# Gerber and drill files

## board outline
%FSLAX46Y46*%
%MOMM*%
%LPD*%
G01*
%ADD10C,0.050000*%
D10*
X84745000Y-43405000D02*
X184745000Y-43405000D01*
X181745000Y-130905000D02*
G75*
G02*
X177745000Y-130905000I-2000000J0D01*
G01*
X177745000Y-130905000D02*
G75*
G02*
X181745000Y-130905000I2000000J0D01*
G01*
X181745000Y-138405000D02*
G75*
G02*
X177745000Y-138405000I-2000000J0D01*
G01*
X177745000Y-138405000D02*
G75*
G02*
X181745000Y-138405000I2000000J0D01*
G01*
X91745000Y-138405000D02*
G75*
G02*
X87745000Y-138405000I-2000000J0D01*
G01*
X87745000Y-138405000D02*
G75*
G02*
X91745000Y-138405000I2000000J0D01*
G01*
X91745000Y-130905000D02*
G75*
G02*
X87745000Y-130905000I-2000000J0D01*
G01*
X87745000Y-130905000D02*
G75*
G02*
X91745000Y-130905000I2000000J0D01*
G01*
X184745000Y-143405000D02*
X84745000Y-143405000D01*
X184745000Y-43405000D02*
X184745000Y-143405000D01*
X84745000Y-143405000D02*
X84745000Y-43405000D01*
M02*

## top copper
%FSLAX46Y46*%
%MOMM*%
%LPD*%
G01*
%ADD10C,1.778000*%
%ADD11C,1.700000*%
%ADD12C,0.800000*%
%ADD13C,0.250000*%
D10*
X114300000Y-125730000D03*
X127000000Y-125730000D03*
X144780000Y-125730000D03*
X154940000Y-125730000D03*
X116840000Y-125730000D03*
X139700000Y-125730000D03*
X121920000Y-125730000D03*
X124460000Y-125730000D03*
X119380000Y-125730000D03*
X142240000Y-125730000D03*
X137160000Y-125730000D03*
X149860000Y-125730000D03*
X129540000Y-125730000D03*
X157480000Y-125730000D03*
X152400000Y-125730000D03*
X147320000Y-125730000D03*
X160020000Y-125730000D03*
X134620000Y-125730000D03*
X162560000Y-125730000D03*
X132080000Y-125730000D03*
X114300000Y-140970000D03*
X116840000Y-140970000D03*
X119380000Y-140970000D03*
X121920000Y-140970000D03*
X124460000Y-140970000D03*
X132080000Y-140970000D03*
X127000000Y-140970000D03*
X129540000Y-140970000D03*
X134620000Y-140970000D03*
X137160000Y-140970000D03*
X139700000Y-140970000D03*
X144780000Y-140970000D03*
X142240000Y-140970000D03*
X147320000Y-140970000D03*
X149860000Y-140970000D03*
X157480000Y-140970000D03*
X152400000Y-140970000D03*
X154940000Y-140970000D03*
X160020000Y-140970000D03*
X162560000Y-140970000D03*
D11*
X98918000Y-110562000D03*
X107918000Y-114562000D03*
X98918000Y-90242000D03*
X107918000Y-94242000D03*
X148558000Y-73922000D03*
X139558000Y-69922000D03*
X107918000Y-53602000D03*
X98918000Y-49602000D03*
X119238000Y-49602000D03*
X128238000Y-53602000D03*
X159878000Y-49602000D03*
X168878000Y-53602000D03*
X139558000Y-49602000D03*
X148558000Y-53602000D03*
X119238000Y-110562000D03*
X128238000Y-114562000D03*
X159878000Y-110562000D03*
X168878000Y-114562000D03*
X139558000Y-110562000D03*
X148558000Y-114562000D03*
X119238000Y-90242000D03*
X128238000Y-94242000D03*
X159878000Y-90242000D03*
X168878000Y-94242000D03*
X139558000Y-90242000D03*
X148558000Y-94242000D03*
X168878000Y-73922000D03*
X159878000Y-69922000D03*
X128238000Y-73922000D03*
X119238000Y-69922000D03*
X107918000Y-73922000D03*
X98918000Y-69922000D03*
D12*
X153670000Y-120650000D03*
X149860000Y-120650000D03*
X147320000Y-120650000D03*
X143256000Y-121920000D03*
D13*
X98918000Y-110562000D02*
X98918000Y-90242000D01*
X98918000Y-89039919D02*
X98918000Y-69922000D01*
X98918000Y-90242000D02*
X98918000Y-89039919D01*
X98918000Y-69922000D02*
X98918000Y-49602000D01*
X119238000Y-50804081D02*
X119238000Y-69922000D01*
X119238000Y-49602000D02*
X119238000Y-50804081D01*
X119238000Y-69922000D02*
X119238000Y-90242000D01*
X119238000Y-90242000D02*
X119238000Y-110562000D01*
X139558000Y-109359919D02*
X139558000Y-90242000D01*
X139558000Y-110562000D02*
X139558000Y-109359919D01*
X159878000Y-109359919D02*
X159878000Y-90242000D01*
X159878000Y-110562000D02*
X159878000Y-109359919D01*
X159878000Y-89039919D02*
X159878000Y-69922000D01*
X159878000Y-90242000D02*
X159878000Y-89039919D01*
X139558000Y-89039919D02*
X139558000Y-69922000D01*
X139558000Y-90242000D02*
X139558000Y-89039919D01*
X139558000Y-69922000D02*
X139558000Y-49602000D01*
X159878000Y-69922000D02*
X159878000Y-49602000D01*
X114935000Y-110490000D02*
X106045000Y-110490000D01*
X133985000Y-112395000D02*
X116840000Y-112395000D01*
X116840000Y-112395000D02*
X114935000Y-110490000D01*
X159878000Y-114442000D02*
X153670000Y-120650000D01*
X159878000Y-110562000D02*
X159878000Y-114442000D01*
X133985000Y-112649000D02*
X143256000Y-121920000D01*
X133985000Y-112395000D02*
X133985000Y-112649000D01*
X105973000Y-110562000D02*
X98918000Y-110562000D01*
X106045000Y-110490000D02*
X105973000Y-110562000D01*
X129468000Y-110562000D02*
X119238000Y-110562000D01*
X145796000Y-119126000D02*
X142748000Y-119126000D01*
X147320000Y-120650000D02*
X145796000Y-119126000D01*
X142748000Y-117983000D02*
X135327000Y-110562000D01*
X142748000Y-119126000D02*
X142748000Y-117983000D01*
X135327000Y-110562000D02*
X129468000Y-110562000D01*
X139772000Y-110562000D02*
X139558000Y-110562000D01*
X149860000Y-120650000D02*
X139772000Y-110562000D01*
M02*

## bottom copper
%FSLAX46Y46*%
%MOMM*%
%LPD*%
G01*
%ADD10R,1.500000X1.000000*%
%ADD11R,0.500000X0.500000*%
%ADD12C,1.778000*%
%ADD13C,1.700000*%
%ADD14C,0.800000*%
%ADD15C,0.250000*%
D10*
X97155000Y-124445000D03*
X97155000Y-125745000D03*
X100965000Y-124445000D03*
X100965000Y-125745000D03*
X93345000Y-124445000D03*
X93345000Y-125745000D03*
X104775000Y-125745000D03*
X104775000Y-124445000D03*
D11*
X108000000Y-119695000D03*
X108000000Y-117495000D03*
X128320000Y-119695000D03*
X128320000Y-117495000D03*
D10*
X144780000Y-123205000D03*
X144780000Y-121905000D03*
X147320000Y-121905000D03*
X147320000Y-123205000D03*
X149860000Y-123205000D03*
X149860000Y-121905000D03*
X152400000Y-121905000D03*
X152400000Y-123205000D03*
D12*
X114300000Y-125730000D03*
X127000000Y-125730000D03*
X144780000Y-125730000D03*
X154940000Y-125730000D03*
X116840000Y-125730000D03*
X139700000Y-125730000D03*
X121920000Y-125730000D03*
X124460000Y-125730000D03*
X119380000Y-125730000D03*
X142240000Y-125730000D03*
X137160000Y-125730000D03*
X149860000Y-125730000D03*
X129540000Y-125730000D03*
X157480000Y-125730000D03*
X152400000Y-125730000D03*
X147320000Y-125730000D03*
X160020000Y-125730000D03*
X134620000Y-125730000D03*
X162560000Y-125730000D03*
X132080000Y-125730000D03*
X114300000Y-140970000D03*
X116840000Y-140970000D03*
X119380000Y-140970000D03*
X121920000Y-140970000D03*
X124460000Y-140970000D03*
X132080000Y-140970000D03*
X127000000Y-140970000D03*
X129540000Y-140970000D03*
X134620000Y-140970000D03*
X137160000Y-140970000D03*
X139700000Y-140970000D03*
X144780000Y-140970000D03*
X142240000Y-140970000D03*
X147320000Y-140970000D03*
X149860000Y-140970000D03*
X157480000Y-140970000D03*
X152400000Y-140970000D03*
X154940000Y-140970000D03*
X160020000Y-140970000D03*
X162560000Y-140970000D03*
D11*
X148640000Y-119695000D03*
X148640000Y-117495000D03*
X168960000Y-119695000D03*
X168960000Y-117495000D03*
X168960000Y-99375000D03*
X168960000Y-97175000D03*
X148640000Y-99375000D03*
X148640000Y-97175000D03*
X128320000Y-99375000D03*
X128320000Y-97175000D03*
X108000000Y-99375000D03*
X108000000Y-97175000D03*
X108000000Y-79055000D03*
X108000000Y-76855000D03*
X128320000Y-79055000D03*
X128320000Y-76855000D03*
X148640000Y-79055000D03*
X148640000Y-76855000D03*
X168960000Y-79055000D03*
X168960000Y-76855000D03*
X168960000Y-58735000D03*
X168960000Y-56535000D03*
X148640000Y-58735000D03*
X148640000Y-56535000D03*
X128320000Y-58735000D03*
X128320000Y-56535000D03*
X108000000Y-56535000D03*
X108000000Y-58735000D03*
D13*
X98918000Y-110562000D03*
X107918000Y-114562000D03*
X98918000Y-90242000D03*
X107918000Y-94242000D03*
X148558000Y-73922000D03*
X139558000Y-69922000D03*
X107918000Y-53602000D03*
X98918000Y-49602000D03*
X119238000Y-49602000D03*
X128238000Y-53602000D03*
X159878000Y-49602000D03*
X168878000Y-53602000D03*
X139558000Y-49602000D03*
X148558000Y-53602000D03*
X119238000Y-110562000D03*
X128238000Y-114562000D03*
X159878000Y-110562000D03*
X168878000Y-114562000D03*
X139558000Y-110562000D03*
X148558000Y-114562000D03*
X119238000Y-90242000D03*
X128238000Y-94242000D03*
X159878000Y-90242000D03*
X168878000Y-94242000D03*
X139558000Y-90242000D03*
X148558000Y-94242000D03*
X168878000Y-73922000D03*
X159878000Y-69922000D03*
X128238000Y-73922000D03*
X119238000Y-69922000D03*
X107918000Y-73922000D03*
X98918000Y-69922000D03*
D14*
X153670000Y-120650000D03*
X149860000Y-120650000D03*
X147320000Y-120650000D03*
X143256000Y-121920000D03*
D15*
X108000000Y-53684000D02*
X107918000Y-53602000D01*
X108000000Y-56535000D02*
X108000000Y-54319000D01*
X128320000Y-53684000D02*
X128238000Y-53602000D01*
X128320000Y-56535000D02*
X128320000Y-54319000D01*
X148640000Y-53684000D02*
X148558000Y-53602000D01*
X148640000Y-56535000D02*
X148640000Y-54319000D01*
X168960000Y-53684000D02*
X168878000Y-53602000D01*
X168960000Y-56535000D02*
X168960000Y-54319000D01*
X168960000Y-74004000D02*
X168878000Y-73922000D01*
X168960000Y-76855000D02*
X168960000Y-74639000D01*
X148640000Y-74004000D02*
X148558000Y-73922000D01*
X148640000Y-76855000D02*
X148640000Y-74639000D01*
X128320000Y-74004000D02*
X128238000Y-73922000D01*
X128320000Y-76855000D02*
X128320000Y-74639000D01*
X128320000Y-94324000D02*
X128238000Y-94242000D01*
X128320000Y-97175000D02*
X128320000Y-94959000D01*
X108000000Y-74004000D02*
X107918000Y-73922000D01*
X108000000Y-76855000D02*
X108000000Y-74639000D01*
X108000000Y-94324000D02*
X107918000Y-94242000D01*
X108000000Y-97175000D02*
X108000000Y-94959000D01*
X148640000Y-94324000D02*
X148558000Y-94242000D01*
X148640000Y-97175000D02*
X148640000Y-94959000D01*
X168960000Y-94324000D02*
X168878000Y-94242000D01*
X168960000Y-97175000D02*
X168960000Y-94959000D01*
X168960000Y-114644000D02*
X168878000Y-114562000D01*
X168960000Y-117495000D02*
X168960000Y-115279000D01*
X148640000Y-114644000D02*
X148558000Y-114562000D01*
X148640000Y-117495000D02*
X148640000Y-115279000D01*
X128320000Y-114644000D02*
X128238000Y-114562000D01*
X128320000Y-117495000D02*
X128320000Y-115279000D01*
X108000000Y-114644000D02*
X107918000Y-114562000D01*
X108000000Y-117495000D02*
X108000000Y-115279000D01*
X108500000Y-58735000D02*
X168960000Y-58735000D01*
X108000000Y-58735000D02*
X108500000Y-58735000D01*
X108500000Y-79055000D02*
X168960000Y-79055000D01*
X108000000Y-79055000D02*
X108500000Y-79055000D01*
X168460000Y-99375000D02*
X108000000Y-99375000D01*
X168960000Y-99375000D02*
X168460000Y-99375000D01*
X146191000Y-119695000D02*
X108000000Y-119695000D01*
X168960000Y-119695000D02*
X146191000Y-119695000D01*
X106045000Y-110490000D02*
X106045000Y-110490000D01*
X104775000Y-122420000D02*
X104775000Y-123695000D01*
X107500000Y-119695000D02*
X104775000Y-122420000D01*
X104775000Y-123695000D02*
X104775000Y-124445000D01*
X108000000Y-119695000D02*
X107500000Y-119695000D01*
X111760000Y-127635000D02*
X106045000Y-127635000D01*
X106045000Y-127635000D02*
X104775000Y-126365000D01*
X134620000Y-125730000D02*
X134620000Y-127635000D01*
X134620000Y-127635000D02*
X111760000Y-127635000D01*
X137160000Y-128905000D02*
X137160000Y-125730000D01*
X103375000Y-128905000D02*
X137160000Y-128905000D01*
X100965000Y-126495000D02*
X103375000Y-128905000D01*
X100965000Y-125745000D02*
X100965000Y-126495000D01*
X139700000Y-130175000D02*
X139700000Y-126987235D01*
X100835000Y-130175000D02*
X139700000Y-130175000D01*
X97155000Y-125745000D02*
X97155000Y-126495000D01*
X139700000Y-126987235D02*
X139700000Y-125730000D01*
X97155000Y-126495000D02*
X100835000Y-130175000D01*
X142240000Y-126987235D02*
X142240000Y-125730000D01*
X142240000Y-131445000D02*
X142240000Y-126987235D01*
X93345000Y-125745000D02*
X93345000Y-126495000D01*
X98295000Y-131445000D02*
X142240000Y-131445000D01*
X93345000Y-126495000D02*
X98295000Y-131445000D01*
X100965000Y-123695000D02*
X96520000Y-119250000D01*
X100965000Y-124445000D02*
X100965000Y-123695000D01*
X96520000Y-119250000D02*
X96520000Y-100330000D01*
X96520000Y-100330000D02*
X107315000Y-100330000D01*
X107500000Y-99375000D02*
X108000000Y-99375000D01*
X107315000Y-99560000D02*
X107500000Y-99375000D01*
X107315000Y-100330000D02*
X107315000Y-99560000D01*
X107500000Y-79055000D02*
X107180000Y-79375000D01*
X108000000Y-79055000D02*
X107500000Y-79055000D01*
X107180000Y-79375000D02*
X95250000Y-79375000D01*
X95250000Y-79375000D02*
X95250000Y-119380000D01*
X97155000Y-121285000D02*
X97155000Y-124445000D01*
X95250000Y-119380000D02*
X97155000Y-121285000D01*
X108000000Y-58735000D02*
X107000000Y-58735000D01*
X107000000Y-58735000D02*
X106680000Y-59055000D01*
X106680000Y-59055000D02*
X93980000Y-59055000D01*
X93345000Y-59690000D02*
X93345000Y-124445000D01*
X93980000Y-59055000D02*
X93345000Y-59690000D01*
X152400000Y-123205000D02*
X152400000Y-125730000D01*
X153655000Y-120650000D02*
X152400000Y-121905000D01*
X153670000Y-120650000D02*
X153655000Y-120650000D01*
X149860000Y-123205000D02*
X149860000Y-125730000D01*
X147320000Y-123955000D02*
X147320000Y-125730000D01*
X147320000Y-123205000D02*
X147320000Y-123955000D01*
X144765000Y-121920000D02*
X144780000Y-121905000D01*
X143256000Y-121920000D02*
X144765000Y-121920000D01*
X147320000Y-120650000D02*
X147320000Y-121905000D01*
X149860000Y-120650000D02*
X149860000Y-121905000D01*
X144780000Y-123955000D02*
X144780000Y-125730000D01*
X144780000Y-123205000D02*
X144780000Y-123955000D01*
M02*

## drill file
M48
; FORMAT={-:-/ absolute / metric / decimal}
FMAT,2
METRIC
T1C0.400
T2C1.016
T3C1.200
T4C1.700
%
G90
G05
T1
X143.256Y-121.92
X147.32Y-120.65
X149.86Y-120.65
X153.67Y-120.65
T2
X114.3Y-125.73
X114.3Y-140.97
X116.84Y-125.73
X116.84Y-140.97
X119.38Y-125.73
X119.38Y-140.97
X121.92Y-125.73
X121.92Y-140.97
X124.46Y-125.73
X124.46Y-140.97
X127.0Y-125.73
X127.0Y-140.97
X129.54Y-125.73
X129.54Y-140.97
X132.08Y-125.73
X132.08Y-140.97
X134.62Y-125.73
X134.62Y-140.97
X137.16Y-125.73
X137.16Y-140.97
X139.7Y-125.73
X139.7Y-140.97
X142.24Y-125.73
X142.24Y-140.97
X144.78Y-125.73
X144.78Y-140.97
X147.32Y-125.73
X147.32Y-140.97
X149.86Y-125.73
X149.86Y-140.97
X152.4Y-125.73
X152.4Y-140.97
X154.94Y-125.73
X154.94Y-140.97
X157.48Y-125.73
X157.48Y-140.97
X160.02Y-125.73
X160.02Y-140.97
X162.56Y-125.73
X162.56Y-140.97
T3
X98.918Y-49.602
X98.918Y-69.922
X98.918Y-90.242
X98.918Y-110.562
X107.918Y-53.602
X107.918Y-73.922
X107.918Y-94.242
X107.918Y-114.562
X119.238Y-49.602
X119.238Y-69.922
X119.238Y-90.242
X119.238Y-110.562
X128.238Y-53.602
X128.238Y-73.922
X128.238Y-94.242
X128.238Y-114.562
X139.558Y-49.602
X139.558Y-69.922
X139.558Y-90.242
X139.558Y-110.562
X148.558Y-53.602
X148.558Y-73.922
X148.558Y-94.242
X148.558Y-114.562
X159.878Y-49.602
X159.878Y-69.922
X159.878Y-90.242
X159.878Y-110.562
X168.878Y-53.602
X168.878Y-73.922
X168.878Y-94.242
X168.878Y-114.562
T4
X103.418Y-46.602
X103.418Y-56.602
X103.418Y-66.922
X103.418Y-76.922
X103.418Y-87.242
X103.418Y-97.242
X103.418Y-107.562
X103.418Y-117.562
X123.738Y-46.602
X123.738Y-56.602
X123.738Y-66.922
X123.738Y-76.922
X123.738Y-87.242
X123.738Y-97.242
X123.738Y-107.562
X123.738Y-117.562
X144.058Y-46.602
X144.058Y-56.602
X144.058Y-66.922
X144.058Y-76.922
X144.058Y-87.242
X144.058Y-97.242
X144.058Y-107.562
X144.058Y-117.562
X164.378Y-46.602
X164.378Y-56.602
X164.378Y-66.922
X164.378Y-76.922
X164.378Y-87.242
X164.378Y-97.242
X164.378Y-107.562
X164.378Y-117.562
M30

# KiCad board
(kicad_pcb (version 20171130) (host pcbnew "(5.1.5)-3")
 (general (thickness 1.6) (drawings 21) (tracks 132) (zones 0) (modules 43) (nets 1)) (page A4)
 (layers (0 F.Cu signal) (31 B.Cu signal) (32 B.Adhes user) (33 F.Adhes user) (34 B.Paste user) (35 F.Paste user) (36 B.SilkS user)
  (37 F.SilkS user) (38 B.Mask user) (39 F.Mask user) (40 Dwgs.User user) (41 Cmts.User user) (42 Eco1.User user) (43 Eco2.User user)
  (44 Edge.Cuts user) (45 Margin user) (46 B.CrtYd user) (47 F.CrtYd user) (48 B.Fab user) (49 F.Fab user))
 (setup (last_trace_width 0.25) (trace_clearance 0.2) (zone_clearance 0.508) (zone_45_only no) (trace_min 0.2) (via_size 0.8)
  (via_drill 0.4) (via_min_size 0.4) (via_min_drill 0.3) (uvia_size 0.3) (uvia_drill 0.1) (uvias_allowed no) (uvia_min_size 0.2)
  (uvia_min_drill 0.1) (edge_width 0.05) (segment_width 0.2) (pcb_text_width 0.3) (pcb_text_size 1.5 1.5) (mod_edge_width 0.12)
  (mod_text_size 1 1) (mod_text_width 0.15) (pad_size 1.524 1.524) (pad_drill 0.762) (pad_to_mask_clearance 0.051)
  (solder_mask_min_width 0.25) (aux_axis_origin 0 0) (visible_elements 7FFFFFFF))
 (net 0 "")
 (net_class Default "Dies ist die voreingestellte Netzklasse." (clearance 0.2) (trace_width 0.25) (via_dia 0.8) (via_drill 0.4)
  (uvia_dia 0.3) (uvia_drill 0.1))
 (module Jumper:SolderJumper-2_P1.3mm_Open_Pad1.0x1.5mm (layer B.Cu) (at 97.155 125.095 90)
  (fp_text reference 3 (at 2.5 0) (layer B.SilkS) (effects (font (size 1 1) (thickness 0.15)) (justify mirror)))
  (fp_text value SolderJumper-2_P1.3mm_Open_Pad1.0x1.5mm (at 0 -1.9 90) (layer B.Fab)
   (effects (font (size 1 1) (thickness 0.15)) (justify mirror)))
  (pad 2 smd rect (at 0.65 0 90) (size 1 1.5) (layers B.Cu B.Mask))
  (pad 1 smd rect (at -0.65 0 90) (size 1 1.5) (layers B.Cu B.Mask)))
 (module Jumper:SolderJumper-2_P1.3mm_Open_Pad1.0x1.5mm (layer B.Cu) (at 100.965 125.095 90)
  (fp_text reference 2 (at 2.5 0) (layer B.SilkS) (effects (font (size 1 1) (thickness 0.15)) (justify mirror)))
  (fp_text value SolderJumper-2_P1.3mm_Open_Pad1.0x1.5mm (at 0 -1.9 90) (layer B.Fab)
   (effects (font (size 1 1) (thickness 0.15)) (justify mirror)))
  (pad 2 smd rect (at 0.65 0 90) (size 1 1.5) (layers B.Cu B.Mask))
  (pad 1 smd rect (at -0.65 0 90) (size 1 1.5) (layers B.Cu B.Mask)))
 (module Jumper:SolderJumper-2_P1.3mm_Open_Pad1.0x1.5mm (layer B.Cu) (at 93.345 125.095 90)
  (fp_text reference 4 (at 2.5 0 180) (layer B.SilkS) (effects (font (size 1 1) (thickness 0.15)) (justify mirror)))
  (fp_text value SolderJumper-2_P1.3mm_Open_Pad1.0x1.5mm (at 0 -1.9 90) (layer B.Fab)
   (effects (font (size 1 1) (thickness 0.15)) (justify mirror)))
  (pad 2 smd rect (at 0.65 0 90) (size 1 1.5) (layers B.Cu B.Mask))
  (pad 1 smd rect (at -0.65 0 90) (size 1 1.5) (layers B.Cu B.Mask)))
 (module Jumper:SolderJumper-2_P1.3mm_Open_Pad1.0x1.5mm (layer B.Cu) (at 104.775 125.095 90)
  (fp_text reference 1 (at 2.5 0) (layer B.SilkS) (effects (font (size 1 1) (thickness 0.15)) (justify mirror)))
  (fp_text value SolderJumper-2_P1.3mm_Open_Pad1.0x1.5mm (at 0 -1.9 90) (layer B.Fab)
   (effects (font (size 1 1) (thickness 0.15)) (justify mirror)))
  (pad 1 smd rect (at -0.65 0 90) (size 1 1.5) (layers B.Cu B.Mask))
  (pad 2 smd rect (at 0.65 0 90) (size 1 1.5) (layers B.Cu B.Mask)))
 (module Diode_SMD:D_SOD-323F (layer B.Cu) (at 108 118.595 90)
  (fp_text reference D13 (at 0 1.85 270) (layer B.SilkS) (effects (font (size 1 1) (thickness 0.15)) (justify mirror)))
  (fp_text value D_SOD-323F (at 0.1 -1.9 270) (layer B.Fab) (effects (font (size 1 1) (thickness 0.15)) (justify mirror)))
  (pad 1 smd rect (at -1.1 0 90) (size 0.5 0.5) (layers B.Cu B.Paste B.Mask))
  (pad 2 smd rect (at 1.1 0 90) (size 0.5 0.5) (layers B.Cu B.Paste B.Mask)))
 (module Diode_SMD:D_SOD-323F (layer B.Cu) (at 128.32 118.595 90)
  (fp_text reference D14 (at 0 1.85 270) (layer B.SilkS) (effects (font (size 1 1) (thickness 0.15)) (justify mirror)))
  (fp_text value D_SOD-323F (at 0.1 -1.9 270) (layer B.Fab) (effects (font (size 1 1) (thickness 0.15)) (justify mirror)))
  (pad 1 smd rect (at -1.1 0 90) (size 0.5 0.5) (layers B.Cu B.Paste B.Mask))
  (pad 2 smd rect (at 1.1 0 90) (size 0.5 0.5) (layers B.Cu B.Paste B.Mask)))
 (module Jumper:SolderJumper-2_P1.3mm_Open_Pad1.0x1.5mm (layer B.Cu) (at 144.78 122.555 270)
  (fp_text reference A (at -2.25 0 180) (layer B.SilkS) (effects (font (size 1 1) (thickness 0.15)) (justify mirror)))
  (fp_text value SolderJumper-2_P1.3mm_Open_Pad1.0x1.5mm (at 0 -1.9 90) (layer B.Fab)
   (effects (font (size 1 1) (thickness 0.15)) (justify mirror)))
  (pad 2 smd rect (at 0.65 0 270) (size 1 1.5) (layers B.Cu B.Mask))
  (pad 1 smd rect (at -0.65 0 270) (size 1 1.5) (layers B.Cu B.Mask)))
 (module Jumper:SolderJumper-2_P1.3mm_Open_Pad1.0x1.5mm (layer B.Cu) (at 147.32 122.555 270)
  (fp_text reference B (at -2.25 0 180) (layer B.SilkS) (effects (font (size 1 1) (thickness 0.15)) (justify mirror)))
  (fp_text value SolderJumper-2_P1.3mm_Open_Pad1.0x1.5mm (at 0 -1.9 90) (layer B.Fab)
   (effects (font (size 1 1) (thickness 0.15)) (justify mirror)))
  (pad 1 smd rect (at -0.65 0 270) (size 1 1.5) (layers B.Cu B.Mask))
  (pad 2 smd rect (at 0.65 0 270) (size 1 1.5) (layers B.Cu B.Mask)))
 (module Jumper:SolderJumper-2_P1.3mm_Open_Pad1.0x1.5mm (layer B.Cu) (at 149.86 122.555 270)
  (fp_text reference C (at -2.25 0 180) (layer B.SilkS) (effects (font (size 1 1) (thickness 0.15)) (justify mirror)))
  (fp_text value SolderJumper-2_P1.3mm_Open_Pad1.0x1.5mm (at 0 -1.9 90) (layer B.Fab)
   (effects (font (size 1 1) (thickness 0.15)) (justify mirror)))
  (pad 2 smd rect (at 0.65 0 270) (size 1 1.5) (layers B.Cu B.Mask))
  (pad 1 smd rect (at -0.65 0 270) (size 1 1.5) (layers B.Cu B.Mask)))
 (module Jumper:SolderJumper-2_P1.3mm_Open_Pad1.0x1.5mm (layer B.Cu) (at 152.4 122.555 270)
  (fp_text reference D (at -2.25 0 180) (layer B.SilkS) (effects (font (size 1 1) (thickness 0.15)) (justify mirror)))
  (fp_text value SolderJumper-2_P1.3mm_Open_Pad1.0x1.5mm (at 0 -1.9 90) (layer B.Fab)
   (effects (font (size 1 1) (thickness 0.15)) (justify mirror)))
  (pad 1 smd rect (at -0.65 0 270) (size 1 1.5) (layers B.Cu B.Mask))
  (pad 2 smd rect (at 0.65 0 270) (size 1 1.5) (layers B.Cu B.Mask)))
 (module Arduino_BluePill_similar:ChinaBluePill (layer F.Cu) (at 162.56 140.97 90)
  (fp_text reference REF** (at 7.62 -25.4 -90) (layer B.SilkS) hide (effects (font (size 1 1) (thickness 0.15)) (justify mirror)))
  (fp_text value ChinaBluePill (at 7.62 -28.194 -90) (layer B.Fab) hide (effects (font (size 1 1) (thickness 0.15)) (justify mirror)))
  (pad GND thru_hole circle (at 15.24 -48.26 180) (size 1.778 1.778) (drill 1.016) (layers *.Cu *.Mask))
  (pad PB10 thru_hole circle (at 15.24 -35.56 180) (size 1.778 1.778) (drill 1.016) (layers *.Cu *.Mask))
  (pad PA3 thru_hole circle (at 15.24 -17.78 180) (size 1.778 1.778) (drill 1.016) (layers *.Cu *.Mask))
  (pad PC15 thru_hole circle (at 15.24 -7.62 180) (size 1.778 1.778) (drill 1.016) (layers *.Cu *.Mask))
  (pad GND thru_hole circle (at 15.24 -45.72 180) (size 1.778 1.778) (drill 1.016) (layers *.Cu *.Mask))
  (pad PA5 thru_hole circle (at 15.24 -22.86 180) (size 1.778 1.778) (drill 1.016) (layers *.Cu *.Mask))
  (pad NRST thru_hole circle (at 15.24 -40.64 180) (size 1.778 1.778) (drill 1.016) (layers *.Cu *.Mask))
  (pad PB11 thru_hole circle (at 15.24 -38.1 180) (size 1.778 1.778) (drill 1.016) (layers *.Cu *.Mask))
  (pad 3V3 thru_hole circle (at 15.24 -43.18 180) (size 1.778 1.778) (drill 1.016) (layers *.Cu *.Mask))
  (pad PA4 thru_hole circle (at 15.24 -20.32 180) (size 1.778 1.778) (drill 1.016) (layers *.Cu *.Mask))
  (pad PA6 thru_hole circle (at 15.24 -25.4 180) (size 1.778 1.778) (drill 1.016) (layers *.Cu *.Mask))
  (pad PA1 thru_hole circle (at 15.24 -12.7 180) (size 1.778 1.778) (drill 1.016) (layers *.Cu *.Mask))
  (pad PB1 thru_hole circle (at 15.24 -33.02 180) (size 1.778 1.778) (drill 1.016) (layers *.Cu *.Mask))
  (pad PC14 thru_hole circle (at 15.24 -5.08 180) (size 1.778 1.778) (drill 1.016) (layers *.Cu *.Mask))
  (pad PA0 thru_hole circle (at 15.24 -10.16 180) (size 1.778 1.778) (drill 1.016) (layers *.Cu *.Mask))
  (pad PA2 thru_hole circle (at 15.24 -15.24 180) (size 1.778 1.778) (drill 1.016) (layers *.Cu *.Mask))
  (pad PC13 thru_hole circle (at 15.24 -2.54 180) (size 1.778 1.778) (drill 1.016) (layers *.Cu *.Mask))
  (pad PA7 thru_hole circle (at 15.24 -27.94 180) (size 1.778 1.778) (drill 1.016) (layers *.Cu *.Mask))
  (pad VBAT thru_hole circle (at 15.24 0 180) (size 1.778 1.778) (drill 1.016) (layers *.Cu *.Mask))
  (pad PB0 thru_hole circle (at 15.24 -30.48 180) (size 1.778 1.778) (drill 1.016) (layers *.Cu *.Mask))
  (pad PB12 thru_hole circle (at 0 -48.26 180) (size 1.778 1.778) (drill 1.016) (layers *.Cu *.Mask))
  (pad PB13 thru_hole circle (at 0 -45.72 180) (size 1.778 1.778) (drill 1.016) (layers *.Cu *.Mask))
  (pad PB14 thru_hole circle (at 0 -43.18 180) (size 1.778 1.778) (drill 1.016) (layers *.Cu *.Mask))
  (pad PB15 thru_hole circle (at 0 -40.64 180) (size 1.778 1.778) (drill 1.016) (layers *.Cu *.Mask))
  (pad PA8 thru_hole circle (at 0 -38.1 180) (size 1.778 1.778) (drill 1.016) (layers *.Cu *.Mask))
  (pad PA11 thru_hole circle (at 0 -30.48 180) (size 1.778 1.778) (drill 1.016) (layers *.Cu *.Mask))
  (pad PA9 thru_hole circle (at 0 -35.56 180) (size 1.778 1.778) (drill 1.016) (layers *.Cu *.Mask))
  (pad PA10 thru_hole circle (at 0 -33.02 180) (size 1.778 1.778) (drill 1.016) (layers *.Cu *.Mask))
  (pad PA12 thru_hole circle (at 0 -27.94 180) (size 1.778 1.778) (drill 1.016) (layers *.Cu *.Mask))
  (pad PA15 thru_hole circle (at 0 -25.4 180) (size 1.778 1.778) (drill 1.016) (layers *.Cu *.Mask))
  (pad PB3 thru_hole circle (at 0 -22.86 180) (size 1.778 1.778) (drill 1.016) (layers *.Cu *.Mask))
  (pad PB5 thru_hole circle (at 0 -17.78 180) (size 1.778 1.778) (drill 1.016) (layers *.Cu *.Mask))
  (pad PB4 thru_hole circle (at 0 -20.32 180) (size 1.778 1.778) (drill 1.016) (layers *.Cu *.Mask))
  (pad PB6 thru_hole circle (at 0 -15.24 180) (size 1.778 1.778) (drill 1.016) (layers *.Cu *.Mask))
  (pad PB7 thru_hole circle (at 0 -12.7 180) (size 1.778 1.778) (drill 1.016) (layers *.Cu *.Mask))
  (pad 5V thru_hole circle (at 0 -5.08 180) (size 1.778 1.778) (drill 1.016) (layers *.Cu *.Mask))
  (pad PB8 thru_hole circle (at 0 -10.16 180) (size 1.778 1.778) (drill 1.016) (layers *.Cu *.Mask))
  (pad PB9 thru_hole circle (at 0 -7.62 180) (size 1.778 1.778) (drill 1.016) (layers *.Cu *.Mask))
  (pad GND thru_hole circle (at 0 -2.54 180) (size 1.778 1.778) (drill 1.016) (layers *.Cu *.Mask))
  (pad 3V3 thru_hole circle (at 0 0 180) (size 1.778 1.778) (drill 1.016) (layers *.Cu *.Mask)))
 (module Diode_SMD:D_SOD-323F (layer B.Cu) (at 148.64 118.595 90)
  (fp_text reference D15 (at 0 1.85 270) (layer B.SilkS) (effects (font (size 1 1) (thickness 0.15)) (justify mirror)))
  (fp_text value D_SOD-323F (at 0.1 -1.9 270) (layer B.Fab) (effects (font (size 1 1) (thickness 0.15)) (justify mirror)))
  (pad 1 smd rect (at -1.1 0 90) (size 0.5 0.5) (layers B.Cu B.Paste B.Mask))
  (pad 2 smd rect (at 1.1 0 90) (size 0.5 0.5) (layers B.Cu B.Paste B.Mask)))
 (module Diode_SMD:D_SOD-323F (layer B.Cu) (at 168.96 118.595 90)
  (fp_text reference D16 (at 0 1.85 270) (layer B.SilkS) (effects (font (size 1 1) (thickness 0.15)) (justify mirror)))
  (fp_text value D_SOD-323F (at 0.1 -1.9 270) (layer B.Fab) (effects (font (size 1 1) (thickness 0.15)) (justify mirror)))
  (pad 1 smd rect (at -1.1 0 90) (size 0.5 0.5) (layers B.Cu B.Paste B.Mask))
  (pad 2 smd rect (at 1.1 0 90) (size 0.5 0.5) (layers B.Cu B.Paste B.Mask)))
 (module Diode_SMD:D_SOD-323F (layer B.Cu) (at 168.96 98.275 90)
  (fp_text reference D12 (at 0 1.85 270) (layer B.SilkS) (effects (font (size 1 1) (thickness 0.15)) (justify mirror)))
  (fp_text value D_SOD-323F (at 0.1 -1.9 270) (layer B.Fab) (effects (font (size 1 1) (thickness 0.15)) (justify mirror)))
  (pad 1 smd rect (at -1.1 0 90) (size 0.5 0.5) (layers B.Cu B.Paste B.Mask))
  (pad 2 smd rect (at 1.1 0 90) (size 0.5 0.5) (layers B.Cu B.Paste B.Mask)))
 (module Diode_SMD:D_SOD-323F (layer B.Cu) (at 148.64 98.275 90)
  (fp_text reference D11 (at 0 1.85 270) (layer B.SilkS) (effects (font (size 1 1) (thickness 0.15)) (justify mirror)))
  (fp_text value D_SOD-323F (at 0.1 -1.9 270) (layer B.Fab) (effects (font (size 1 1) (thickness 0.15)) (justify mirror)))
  (pad 1 smd rect (at -1.1 0 90) (size 0.5 0.5) (layers B.Cu B.Paste B.Mask))
  (pad 2 smd rect (at 1.1 0 90) (size 0.5 0.5) (layers B.Cu B.Paste B.Mask)))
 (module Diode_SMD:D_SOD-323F (layer B.Cu) (at 128.32 98.275 90)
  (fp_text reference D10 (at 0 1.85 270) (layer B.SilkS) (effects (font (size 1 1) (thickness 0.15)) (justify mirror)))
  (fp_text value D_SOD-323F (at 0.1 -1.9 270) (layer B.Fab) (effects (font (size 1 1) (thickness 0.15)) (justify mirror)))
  (pad 1 smd rect (at -1.1 0 90) (size 0.5 0.5) (layers B.Cu B.Paste B.Mask))
  (pad 2 smd rect (at 1.1 0 90) (size 0.5 0.5) (layers B.Cu B.Paste B.Mask)))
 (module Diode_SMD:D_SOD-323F (layer B.Cu) (at 108 98.275 90)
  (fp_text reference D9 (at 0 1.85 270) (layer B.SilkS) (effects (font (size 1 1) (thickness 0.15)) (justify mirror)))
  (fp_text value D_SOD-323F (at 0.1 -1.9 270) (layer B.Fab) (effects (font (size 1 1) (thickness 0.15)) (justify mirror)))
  (pad 1 smd rect (at -1.1 0 90) (size 0.5 0.5) (layers B.Cu B.Paste B.Mask))
  (pad 2 smd rect (at 1.1 0 90) (size 0.5 0.5) (layers B.Cu B.Paste B.Mask)))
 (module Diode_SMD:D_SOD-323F (layer B.Cu) (at 108 77.955 90)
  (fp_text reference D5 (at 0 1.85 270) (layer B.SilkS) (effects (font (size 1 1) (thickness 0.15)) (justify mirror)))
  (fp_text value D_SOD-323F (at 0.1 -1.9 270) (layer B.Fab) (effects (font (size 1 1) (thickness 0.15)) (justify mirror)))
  (pad 1 smd rect (at -1.1 0 90) (size 0.5 0.5) (layers B.Cu B.Paste B.Mask))
  (pad 2 smd rect (at 1.1 0 90) (size 0.5 0.5) (layers B.Cu B.Paste B.Mask)))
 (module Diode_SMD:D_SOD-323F (layer B.Cu) (at 128.32 77.955 90)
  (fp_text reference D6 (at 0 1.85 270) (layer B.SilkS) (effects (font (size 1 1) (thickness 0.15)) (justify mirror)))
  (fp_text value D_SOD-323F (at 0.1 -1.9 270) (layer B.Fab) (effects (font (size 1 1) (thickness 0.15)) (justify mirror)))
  (pad 1 smd rect (at -1.1 0 90) (size 0.5 0.5) (layers B.Cu B.Paste B.Mask))
  (pad 2 smd rect (at 1.1 0 90) (size 0.5 0.5) (layers B.Cu B.Paste B.Mask)))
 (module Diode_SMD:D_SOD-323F (layer B.Cu) (at 148.64 77.955 90)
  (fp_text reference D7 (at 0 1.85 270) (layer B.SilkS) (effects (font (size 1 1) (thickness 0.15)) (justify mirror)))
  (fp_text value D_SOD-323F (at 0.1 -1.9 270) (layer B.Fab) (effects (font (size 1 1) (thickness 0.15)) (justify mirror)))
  (pad 1 smd rect (at -1.1 0 90) (size 0.5 0.5) (layers B.Cu B.Paste B.Mask))
  (pad 2 smd rect (at 1.1 0 90) (size 0.5 0.5) (layers B.Cu B.Paste B.Mask)))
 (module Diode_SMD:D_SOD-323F (layer B.Cu) (at 168.96 77.955 90)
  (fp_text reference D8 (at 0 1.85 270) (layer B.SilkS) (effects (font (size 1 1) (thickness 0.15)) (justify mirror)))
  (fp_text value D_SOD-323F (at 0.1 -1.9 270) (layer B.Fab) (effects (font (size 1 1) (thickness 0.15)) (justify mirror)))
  (pad 1 smd rect (at -1.1 0 90) (size 0.5 0.5) (layers B.Cu B.Paste B.Mask))
  (pad 2 smd rect (at 1.1 0 90) (size 0.5 0.5) (layers B.Cu B.Paste B.Mask)))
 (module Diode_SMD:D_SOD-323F (layer B.Cu) (at 168.96 57.635 90)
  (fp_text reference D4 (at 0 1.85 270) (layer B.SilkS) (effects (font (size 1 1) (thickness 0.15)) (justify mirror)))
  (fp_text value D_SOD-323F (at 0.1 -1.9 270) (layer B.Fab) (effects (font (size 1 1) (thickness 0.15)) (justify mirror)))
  (pad 1 smd rect (at -1.1 0 90) (size 0.5 0.5) (layers B.Cu B.Paste B.Mask))
  (pad 2 smd rect (at 1.1 0 90) (size 0.5 0.5) (layers B.Cu B.Paste B.Mask)))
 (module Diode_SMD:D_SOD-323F (layer B.Cu) (at 148.64 57.635 90)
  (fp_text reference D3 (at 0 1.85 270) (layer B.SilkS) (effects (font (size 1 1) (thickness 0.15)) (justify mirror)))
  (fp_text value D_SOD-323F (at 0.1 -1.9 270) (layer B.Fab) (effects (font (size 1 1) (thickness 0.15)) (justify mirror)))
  (pad 1 smd rect (at -1.1 0 90) (size 0.5 0.5) (layers B.Cu B.Paste B.Mask))
  (pad 2 smd rect (at 1.1 0 90) (size 0.5 0.5) (layers B.Cu B.Paste B.Mask)))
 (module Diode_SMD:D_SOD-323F (layer B.Cu) (at 128.32 57.635 90)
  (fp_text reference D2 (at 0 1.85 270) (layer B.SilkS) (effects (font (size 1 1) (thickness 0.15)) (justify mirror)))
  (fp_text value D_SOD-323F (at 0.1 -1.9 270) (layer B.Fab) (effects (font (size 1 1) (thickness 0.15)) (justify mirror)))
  (pad 1 smd rect (at -1.1 0 90) (size 0.5 0.5) (layers B.Cu B.Paste B.Mask))
  (pad 2 smd rect (at 1.1 0 90) (size 0.5 0.5) (layers B.Cu B.Paste B.Mask)))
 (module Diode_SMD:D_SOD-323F (layer B.Cu) (at 108 57.635 90)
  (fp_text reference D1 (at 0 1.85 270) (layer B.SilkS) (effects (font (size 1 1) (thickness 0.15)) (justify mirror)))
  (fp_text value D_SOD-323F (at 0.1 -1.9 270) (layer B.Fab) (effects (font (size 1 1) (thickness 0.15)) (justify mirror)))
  (pad 2 smd rect (at 1.1 0 90) (size 0.5 0.5) (layers B.Cu B.Paste B.Mask))
  (pad 1 smd rect (at -1.1 0 90) (size 0.5 0.5) (layers B.Cu B.Paste B.Mask)))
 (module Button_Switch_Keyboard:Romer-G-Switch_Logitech (layer F.Cu) (at 103.418 112.562)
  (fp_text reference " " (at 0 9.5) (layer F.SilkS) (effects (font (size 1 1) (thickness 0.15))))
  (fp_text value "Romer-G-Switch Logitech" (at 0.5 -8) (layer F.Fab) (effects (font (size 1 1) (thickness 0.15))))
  (pad 1 thru_hole circle (at -4.5 -2) (size 1.7 1.7) (drill 1.2) (layers *.Cu *.Mask))
  (pad 2 thru_hole circle (at 4.5 2) (size 1.7 1.7) (drill 1.2) (layers *.Cu *.Mask))
  (pad "" np_thru_hole circle (at 0 -5) (size 1.7 1.7) (drill 1.7) (layers *.Cu *.Mask))
  (pad "" np_thru_hole circle (at 0 5) (size 1.7 1.7) (drill 1.7) (layers *.Cu *.Mask)))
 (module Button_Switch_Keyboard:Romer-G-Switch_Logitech (layer F.Cu) (at 103.418 92.242)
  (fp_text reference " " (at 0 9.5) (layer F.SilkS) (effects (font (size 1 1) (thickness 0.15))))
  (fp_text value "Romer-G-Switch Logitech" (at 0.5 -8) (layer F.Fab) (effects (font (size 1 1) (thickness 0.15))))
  (pad 1 thru_hole circle (at -4.5 -2) (size 1.7 1.7) (drill 1.2) (layers *.Cu *.Mask))
  (pad 2 thru_hole circle (at 4.5 2) (size 1.7 1.7) (drill 1.2) (layers *.Cu *.Mask))
  (pad "" np_thru_hole circle (at 0 -5) (size 1.7 1.7) (drill 1.7) (layers *.Cu *.Mask))
  (pad "" np_thru_hole circle (at 0 5) (size 1.7 1.7) (drill 1.7) (layers *.Cu *.Mask)))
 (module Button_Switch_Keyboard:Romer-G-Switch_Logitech (layer F.Cu) (at 144.058 71.922)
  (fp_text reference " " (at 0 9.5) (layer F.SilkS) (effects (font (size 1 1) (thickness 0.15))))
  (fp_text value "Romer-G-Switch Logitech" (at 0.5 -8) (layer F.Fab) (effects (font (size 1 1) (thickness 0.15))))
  (pad "" np_thru_hole circle (at 0 5) (size 1.7 1.7) (drill 1.7) (layers *.Cu *.Mask))
  (pad "" np_thru_hole circle (at 0 -5) (size 1.7 1.7) (drill 1.7) (layers *.Cu *.Mask))
  (pad 2 thru_hole circle (at 4.5 2) (size 1.7 1.7) (drill 1.2) (layers *.Cu *.Mask))
  (pad 1 thru_hole circle (at -4.5 -2) (size 1.7 1.7) (drill 1.2) (layers *.Cu *.Mask)))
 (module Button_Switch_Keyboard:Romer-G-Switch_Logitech (layer F.Cu) (at 103.418 51.602)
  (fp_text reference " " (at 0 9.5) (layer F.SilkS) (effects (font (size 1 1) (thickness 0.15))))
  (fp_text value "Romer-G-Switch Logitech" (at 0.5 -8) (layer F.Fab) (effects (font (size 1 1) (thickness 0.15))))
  (pad "" np_thru_hole circle (at 0 5) (size 1.7 1.7) (drill 1.7) (layers *.Cu *.Mask))
  (pad "" np_thru_hole circle (at 0 -5) (size 1.7 1.7) (drill 1.7) (layers *.Cu *.Mask))
  (pad 2 thru_hole circle (at 4.5 2) (size 1.7 1.7) (drill 1.2) (layers *.Cu *.Mask))
  (pad 1 thru_hole circle (at -4.5 -2) (size 1.7 1.7) (drill 1.2) (layers *.Cu *.Mask)))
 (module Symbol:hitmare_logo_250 (layer B.Cu) (at 140.335 80.01 180)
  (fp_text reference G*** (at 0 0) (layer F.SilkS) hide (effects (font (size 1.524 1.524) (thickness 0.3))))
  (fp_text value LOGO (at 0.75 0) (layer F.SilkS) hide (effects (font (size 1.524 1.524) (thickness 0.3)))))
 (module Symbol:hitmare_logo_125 (layer F.Cu) (at 179.705 116.205)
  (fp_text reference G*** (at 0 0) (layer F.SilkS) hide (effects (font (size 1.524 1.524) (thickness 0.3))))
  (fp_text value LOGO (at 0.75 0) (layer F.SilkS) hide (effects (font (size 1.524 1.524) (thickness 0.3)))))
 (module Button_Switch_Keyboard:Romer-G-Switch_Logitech (layer F.Cu) (at 123.738 51.602)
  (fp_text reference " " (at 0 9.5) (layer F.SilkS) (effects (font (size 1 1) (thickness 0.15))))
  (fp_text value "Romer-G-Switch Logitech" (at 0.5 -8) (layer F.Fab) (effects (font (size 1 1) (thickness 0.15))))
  (pad 1 thru_hole circle (at -4.5 -2) (size 1.7 1.7) (drill 1.2) (layers *.Cu *.Mask))
  (pad 2 thru_hole circle (at 4.5 2) (size 1.7 1.7) (drill 1.2) (layers *.Cu *.Mask))
  (pad "" np_thru_hole circle (at 0 -5) (size 1.7 1.7) (drill 1.7) (layers *.Cu *.Mask))
  (pad "" np_thru_hole circle (at 0 5) (size 1.7 1.7) (drill 1.7) (layers *.Cu *.Mask)))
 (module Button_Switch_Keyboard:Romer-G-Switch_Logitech (layer F.Cu) (at 164.378 51.602)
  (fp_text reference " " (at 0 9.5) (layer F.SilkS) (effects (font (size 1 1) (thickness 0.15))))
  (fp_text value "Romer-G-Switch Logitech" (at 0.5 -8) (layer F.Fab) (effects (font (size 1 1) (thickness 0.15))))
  (pad 1 thru_hole circle (at -4.5 -2) (size 1.7 1.7) (drill 1.2) (layers *.Cu *.Mask))
  (pad 2 thru_hole circle (at 4.5 2) (size 1.7 1.7) (drill 1.2) (layers *.Cu *.Mask))
  (pad "" np_thru_hole circle (at 0 -5) (size 1.7 1.7) (drill 1.7) (layers *.Cu *.Mask))
  (pad "" np_thru_hole circle (at 0 5) (size 1.7 1.7) (drill 1.7) (layers *.Cu *.Mask)))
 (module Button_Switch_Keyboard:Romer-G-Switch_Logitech (layer F.Cu) (at 144.058 51.602)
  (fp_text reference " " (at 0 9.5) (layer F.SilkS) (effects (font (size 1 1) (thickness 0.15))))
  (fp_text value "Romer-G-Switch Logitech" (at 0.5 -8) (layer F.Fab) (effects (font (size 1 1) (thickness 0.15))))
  (pad 1 thru_hole circle (at -4.5 -2) (size 1.7 1.7) (drill 1.2) (layers *.Cu *.Mask))
  (pad 2 thru_hole circle (at 4.5 2) (size 1.7 1.7) (drill 1.2) (layers *.Cu *.Mask))
  (pad "" np_thru_hole circle (at 0 -5) (size 1.7 1.7) (drill 1.7) (layers *.Cu *.Mask))
  (pad "" np_thru_hole circle (at 0 5) (size 1.7 1.7) (drill 1.7) (layers *.Cu *.Mask)))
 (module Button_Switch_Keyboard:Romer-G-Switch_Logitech (layer F.Cu) (at 123.738 112.562)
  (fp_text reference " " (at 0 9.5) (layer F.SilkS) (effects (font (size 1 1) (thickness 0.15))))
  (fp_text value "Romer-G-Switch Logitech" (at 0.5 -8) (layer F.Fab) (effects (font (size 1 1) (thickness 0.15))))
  (pad 1 thru_hole circle (at -4.5 -2) (size 1.7 1.7) (drill 1.2) (layers *.Cu *.Mask))
  (pad 2 thru_hole circle (at 4.5 2) (size 1.7 1.7) (drill 1.2) (layers *.Cu *.Mask))
  (pad "" np_thru_hole circle (at 0 -5) (size 1.7 1.7) (drill 1.7) (layers *.Cu *.Mask))
  (pad "" np_thru_hole circle (at 0 5) (size 1.7 1.7) (drill 1.7) (layers *.Cu *.Mask)))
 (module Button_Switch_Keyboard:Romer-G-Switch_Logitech (layer F.Cu) (at 164.378 112.562)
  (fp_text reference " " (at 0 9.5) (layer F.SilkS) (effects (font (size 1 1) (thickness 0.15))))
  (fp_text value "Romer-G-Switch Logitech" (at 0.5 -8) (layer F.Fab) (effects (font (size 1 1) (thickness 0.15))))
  (pad 1 thru_hole circle (at -4.5 -2) (size 1.7 1.7) (drill 1.2) (layers *.Cu *.Mask))
  (pad 2 thru_hole circle (at 4.5 2) (size 1.7 1.7) (drill 1.2) (layers *.Cu *.Mask))
  (pad "" np_thru_hole circle (at 0 -5) (size 1.7 1.7) (drill 1.7) (layers *.Cu *.Mask))
  (pad "" np_thru_hole circle (at 0 5) (size 1.7 1.7) (drill 1.7) (layers *.Cu *.Mask)))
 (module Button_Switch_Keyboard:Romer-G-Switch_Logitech (layer F.Cu) (at 144.058 112.562)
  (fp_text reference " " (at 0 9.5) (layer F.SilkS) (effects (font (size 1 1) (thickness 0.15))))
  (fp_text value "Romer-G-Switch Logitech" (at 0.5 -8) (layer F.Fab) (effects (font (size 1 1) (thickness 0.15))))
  (pad 1 thru_hole circle (at -4.5 -2) (size 1.7 1.7) (drill 1.2) (layers *.Cu *.Mask))
  (pad 2 thru_hole circle (at 4.5 2) (size 1.7 1.7) (drill 1.2) (layers *.Cu *.Mask))
  (pad "" np_thru_hole circle (at 0 -5) (size 1.7 1.7) (drill 1.7) (layers *.Cu *.Mask))
  (pad "" np_thru_hole circle (at 0 5) (size 1.7 1.7) (drill 1.7) (layers *.Cu *.Mask)))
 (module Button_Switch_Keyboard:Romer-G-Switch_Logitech (layer F.Cu) (at 123.738 92.242)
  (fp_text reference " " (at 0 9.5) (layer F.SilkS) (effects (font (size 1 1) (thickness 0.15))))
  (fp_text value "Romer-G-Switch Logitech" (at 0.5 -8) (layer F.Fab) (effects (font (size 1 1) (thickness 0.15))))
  (pad 1 thru_hole circle (at -4.5 -2) (size 1.7 1.7) (drill 1.2) (layers *.Cu *.Mask))
  (pad 2 thru_hole circle (at 4.5 2) (size 1.7 1.7) (drill 1.2) (layers *.Cu *.Mask))
  (pad "" np_thru_hole circle (at 0 -5) (size 1.7 1.7) (drill 1.7) (layers *.Cu *.Mask))
  (pad "" np_thru_hole circle (at 0 5) (size 1.7 1.7) (drill 1.7) (layers *.Cu *.Mask)))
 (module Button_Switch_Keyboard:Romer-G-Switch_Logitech (layer F.Cu) (at 164.378 92.242)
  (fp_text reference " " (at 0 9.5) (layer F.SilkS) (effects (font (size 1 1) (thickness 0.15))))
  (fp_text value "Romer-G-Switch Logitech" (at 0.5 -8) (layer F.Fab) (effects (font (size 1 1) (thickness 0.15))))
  (pad 1 thru_hole circle (at -4.5 -2) (size 1.7 1.7) (drill 1.2) (layers *.Cu *.Mask))
  (pad 2 thru_hole circle (at 4.5 2) (size 1.7 1.7) (drill 1.2) (layers *.Cu *.Mask))
  (pad "" np_thru_hole circle (at 0 -5) (size 1.7 1.7) (drill 1.7) (layers *.Cu *.Mask))
  (pad "" np_thru_hole circle (at 0 5) (size 1.7 1.7) (drill 1.7) (layers *.Cu *.Mask)))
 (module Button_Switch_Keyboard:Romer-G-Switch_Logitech (layer F.Cu) (at 144.058 92.242)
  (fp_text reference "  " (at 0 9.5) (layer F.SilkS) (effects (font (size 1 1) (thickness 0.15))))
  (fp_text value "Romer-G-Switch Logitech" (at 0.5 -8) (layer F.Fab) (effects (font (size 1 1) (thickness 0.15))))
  (pad 1 thru_hole circle (at -4.5 -2) (size 1.7 1.7) (drill 1.2) (layers *.Cu *.Mask))
  (pad 2 thru_hole circle (at 4.5 2) (size 1.7 1.7) (drill 1.2) (layers *.Cu *.Mask))
  (pad "" np_thru_hole circle (at 0 -5) (size 1.7 1.7) (drill 1.7) (layers *.Cu *.Mask))
  (pad "" np_thru_hole circle (at 0 5) (size 1.7 1.7) (drill 1.7) (layers *.Cu *.Mask)))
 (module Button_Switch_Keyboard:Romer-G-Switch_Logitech (layer F.Cu) (at 164.378 71.922)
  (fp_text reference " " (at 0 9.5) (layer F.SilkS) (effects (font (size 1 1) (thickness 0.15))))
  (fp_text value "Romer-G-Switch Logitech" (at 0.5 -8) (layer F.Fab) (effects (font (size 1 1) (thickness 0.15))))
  (pad "" np_thru_hole circle (at 0 5) (size 1.7 1.7) (drill 1.7) (layers *.Cu *.Mask))
  (pad "" np_thru_hole circle (at 0 -5) (size 1.7 1.7) (drill 1.7) (layers *.Cu *.Mask))
  (pad 2 thru_hole circle (at 4.5 2) (size 1.7 1.7) (drill 1.2) (layers *.Cu *.Mask))
  (pad 1 thru_hole circle (at -4.5 -2) (size 1.7 1.7) (drill 1.2) (layers *.Cu *.Mask)))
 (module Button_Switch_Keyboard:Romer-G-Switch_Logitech (layer F.Cu) (at 123.738 71.922)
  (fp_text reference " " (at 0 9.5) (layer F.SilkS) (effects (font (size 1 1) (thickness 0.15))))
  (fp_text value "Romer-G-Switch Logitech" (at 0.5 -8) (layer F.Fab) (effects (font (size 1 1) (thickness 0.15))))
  (pad "" np_thru_hole circle (at 0 5) (size 1.7 1.7) (drill 1.7) (layers *.Cu *.Mask))
  (pad "" np_thru_hole circle (at 0 -5) (size 1.7 1.7) (drill 1.7) (layers *.Cu *.Mask))
  (pad 2 thru_hole circle (at 4.5 2) (size 1.7 1.7) (drill 1.2) (layers *.Cu *.Mask))
  (pad 1 thru_hole circle (at -4.5 -2) (size 1.7 1.7) (drill 1.2) (layers *.Cu *.Mask)))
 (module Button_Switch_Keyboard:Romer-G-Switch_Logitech (layer F.Cu) (at 103.418 71.922)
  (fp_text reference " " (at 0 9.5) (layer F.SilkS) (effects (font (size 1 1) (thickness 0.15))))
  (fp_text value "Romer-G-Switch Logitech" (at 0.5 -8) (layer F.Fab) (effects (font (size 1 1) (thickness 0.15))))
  (pad "" np_thru_hole circle (at 0 5) (size 1.7 1.7) (drill 1.7) (layers *.Cu *.Mask))
  (pad "" np_thru_hole circle (at 0 -5) (size 1.7 1.7) (drill 1.7) (layers *.Cu *.Mask))
  (pad 2 thru_hole circle (at 4.5 2) (size 1.7 1.7) (drill 1.2) (layers *.Cu *.Mask))
  (pad 1 thru_hole circle (at -4.5 -2) (size 1.7 1.7) (drill 1.2) (layers *.Cu *.Mask)))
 (gr_line (start 84.745 43.405) (end 184.745 43.405) (layer Edge.Cuts) (width 0.05))
 (gr_circle (center 179.745 130.905) (end 181.745 130.905) (layer Edge.Cuts) (width 0.05))
 (gr_circle (center 179.745 138.405) (end 181.745 138.405) (layer Edge.Cuts) (width 0.05))
 (gr_circle (center 89.745 138.405) (end 91.745 138.405) (layer Edge.Cuts) (width 0.05))
 (gr_circle (center 89.745 130.905) (end 91.745 130.905) (layer Edge.Cuts) (width 0.05))
 (gr_line (start 184.745 143.405) (end 84.745 143.405) (layer Edge.Cuts) (width 0.05))
 (gr_line (start 184.745 43.405) (end 184.745 143.405) (layer Edge.Cuts) (width 0.05))
 (gr_line (start 84.745 143.405) (end 84.745 43.405) (layer Edge.Cuts) (width 0.05))
 (segment (start 98.918 110.562) (end 98.918 90.242) (width 0.25) (layer F.Cu) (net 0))
 (segment (start 98.918 89.039919) (end 98.918 69.922) (width 0.25) (layer F.Cu) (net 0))
 (segment (start 98.918 90.242) (end 98.918 89.039919) (width 0.25) (layer F.Cu) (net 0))
 (segment (start 98.918 69.922) (end 98.918 49.602) (width 0.25) (layer F.Cu) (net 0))
 (segment (start 119.238 50.804081) (end 119.238 69.922) (width 0.25) (layer F.Cu) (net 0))
 (segment (start 119.238 49.602) (end 119.238 50.804081) (width 0.25) (layer F.Cu) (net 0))
 (segment (start 119.238 69.922) (end 119.238 90.242) (width 0.25) (layer F.Cu) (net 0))
 (segment (start 119.238 90.242) (end 119.238 110.562) (width 0.25) (layer F.Cu) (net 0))
 (segment (start 139.558 109.359919) (end 139.558 90.242) (width 0.25) (layer F.Cu) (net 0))
 (segment (start 139.558 110.562) (end 139.558 109.359919) (width 0.25) (layer F.Cu) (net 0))
 (segment (start 159.878 109.359919) (end 159.878 90.242) (width 0.25) (layer F.Cu) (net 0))
 (segment (start 159.878 110.562) (end 159.878 109.359919) (width 0.25) (layer F.Cu) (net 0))
 (segment (start 159.878 89.039919) (end 159.878 69.922) (width 0.25) (layer F.Cu) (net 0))
 (segment (start 159.878 90.242) (end 159.878 89.039919) (width 0.25) (layer F.Cu) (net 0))
 (segment (start 139.558 89.039919) (end 139.558 69.922) (width 0.25) (layer F.Cu) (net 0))
 (segment (start 139.558 90.242) (end 139.558 89.039919) (width 0.25) (layer F.Cu) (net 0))
 (segment (start 139.558 69.922) (end 139.558 49.602) (width 0.25) (layer F.Cu) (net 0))
 (segment (start 159.878 69.922) (end 159.878 49.602) (width 0.25) (layer F.Cu) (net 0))
 (segment (start 108 53.684) (end 107.918 53.602) (width 0.25) (layer B.Cu) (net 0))
 (segment (start 108 56.535) (end 108 54.319) (width 0.25) (layer B.Cu) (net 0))
 (segment (start 128.32 53.684) (end 128.238 53.602) (width 0.25) (layer B.Cu) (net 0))
 (segment (start 128.32 56.535) (end 128.32 54.319) (width 0.25) (layer B.Cu) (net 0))
 (segment (start 148.64 53.684) (end 148.558 53.602) (width 0.25) (layer B.Cu) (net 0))
 (segment (start 148.64 56.535) (end 148.64 54.319) (width 0.25) (layer B.Cu) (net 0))
 (segment (start 168.96 53.684) (end 168.878 53.602) (width 0.25) (layer B.Cu) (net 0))
 (segment (start 168.96 56.535) (end 168.96 54.319) (width 0.25) (layer B.Cu) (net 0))
 (segment (start 168.96 74.004) (end 168.878 73.922) (width 0.25) (layer B.Cu) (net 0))
 (segment (start 168.96 76.855) (end 168.96 74.639) (width 0.25) (layer B.Cu) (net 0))
 (segment (start 148.64 74.004) (end 148.558 73.922) (width 0.25) (layer B.Cu) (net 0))
 (segment (start 148.64 76.855) (end 148.64 74.639) (width 0.25) (layer B.Cu) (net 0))
 (segment (start 128.32 74.004) (end 128.238 73.922) (width 0.25) (layer B.Cu) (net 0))
 (segment (start 128.32 76.855) (end 128.32 74.639) (width 0.25) (layer B.Cu) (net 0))
 (segment (start 128.32 94.324) (end 128.238 94.242) (width 0.25) (layer B.Cu) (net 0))
 (segment (start 128.32 97.175) (end 128.32 94.959) (width 0.25) (layer B.Cu) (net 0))
 (segment (start 108 74.004) (end 107.918 73.922) (width 0.25) (layer B.Cu) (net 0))
 (segment (start 108 76.855) (end 108 74.639) (width 0.25) (layer B.Cu) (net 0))
 (segment (start 108 94.324) (end 107.918 94.242) (width 0.25) (layer B.Cu) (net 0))
 (segment (start 108 97.175) (end 108 94.959) (width 0.25) (layer B.Cu) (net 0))
 (segment (start 148.64 94.324) (end 148.558 94.242) (width 0.25) (layer B.Cu) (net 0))
 (segment (start 148.64 97.175) (end 148.64 94.959) (width 0.25) (layer B.Cu) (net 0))
 (segment (start 168.96 94.324) (end 168.878 94.242) (width 0.25) (layer B.Cu) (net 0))
 (segment (start 168.96 97.175) (end 168.96 94.959) (width 0.25) (layer B.Cu) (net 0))
 (segment (start 168.96 114.644) (end 168.878 114.562) (width 0.25) (layer B.Cu) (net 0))
 (segment (start 168.96 117.495) (end 168.96 115.279) (width 0.25) (layer B.Cu) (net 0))
 (segment (start 148.64 114.644) (end 148.558 114.562) (width 0.25) (layer B.Cu) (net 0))
 (segment (start 148.64 117.495) (end 148.64 115.279) (width 0.25) (layer B.Cu) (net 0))
 (segment (start 128.32 114.644) (end 128.238 114.562) (width 0.25) (layer B.Cu) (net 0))
 (segment (start 128.32 117.495) (end 128.32 115.279) (width 0.25) (layer B.Cu) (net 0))
 (segment (start 108 114.644) (end 107.918 114.562) (width 0.25) (layer B.Cu) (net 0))
 (segment (start 108 117.495) (end 108 115.279) (width 0.25) (layer B.Cu) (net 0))
 (segment (start 108.5 58.735) (end 168.96 58.735) (width 0.25) (layer B.Cu) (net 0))
 (segment (start 108 58.735) (end 108.5 58.735) (width 0.25) (layer B.Cu) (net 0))
 (segment (start 108.5 79.055) (end 168.96 79.055) (width 0.25) (layer B.Cu) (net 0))
 (segment (start 108 79.055) (end 108.5 79.055) (width 0.25) (layer B.Cu) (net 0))
 (segment (start 168.46 99.375) (end 108 99.375) (width 0.25) (layer B.Cu) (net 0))
 (segment (start 168.96 99.375) (end 168.46 99.375) (width 0.25) (layer B.Cu) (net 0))
 (segment (start 146.191 119.695) (end 108 119.695) (width 0.25) (layer B.Cu) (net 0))
 (segment (start 168.96 119.695) (end 146.191 119.695) (width 0.25) (layer B.Cu) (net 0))
 (segment (start 106.045 110.49) (end 106.045 110.49) (width 0.25) (layer B.Cu) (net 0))
 (segment (start 114.935 110.49) (end 106.045 110.49) (width 0.25) (layer F.Cu) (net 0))
 (segment (start 133.985 112.395) (end 116.84 112.395) (width 0.25) (layer F.Cu) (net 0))
 (segment (start 116.84 112.395) (end 114.935 110.49) (width 0.25) (layer F.Cu) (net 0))
 (via (at 153.67 120.65) (size 0.8) (drill 0.4) (layers F.Cu B.Cu) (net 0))
 (segment (start 104.775 122.42) (end 104.775 123.695) (width 0.25) (layer B.Cu) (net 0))
 (segment (start 107.5 119.695) (end 104.775 122.42) (width 0.25) (layer B.Cu) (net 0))
 (segment (start 104.775 123.695) (end 104.775 124.445) (width 0.25) (layer B.Cu) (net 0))
 (segment (start 108 119.695) (end 107.5 119.695) (width 0.25) (layer B.Cu) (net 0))
 (segment (start 111.76 127.635) (end 106.045 127.635) (width 0.25) (layer B.Cu) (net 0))
 (segment (start 106.045 127.635) (end 104.775 126.365) (width 0.25) (layer B.Cu) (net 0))
 (segment (start 134.62 125.73) (end 134.62 127.635) (width 0.25) (layer B.Cu) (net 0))
 (segment (start 134.62 127.635) (end 111.76 127.635) (width 0.25) (layer B.Cu) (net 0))
 (segment (start 137.16 128.905) (end 137.16 125.73) (width 0.25) (layer B.Cu) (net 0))
 (segment (start 103.375 128.905) (end 137.16 128.905) (width 0.25) (layer B.Cu) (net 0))
 (segment (start 100.965 126.495) (end 103.375 128.905) (width 0.25) (layer B.Cu) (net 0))
 (segment (start 100.965 125.745) (end 100.965 126.495) (width 0.25) (layer B.Cu) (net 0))
 (segment (start 139.7 130.175) (end 139.7 126.987235) (width 0.25) (layer B.Cu) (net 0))
 (segment (start 100.835 130.175) (end 139.7 130.175) (width 0.25) (layer B.Cu) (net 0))
 (segment (start 97.155 125.745) (end 97.155 126.495) (width 0.25) (layer B.Cu) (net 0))
 (segment (start 139.7 126.987235) (end 139.7 125.73) (width 0.25) (layer B.Cu) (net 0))
 (segment (start 97.155 126.495) (end 100.835 130.175) (width 0.25) (layer B.Cu) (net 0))
 (segment (start 142.24 126.987235) (end 142.24 125.73) (width 0.25) (layer B.Cu) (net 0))
 (segment (start 142.24 131.445) (end 142.24 126.987235) (width 0.25) (layer B.Cu) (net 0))
 (segment (start 93.345 125.745) (end 93.345 126.495) (width 0.25) (layer B.Cu) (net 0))
 (segment (start 98.295 131.445) (end 142.24 131.445) (width 0.25) (layer B.Cu) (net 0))
 (segment (start 93.345 126.495) (end 98.295 131.445) (width 0.25) (layer B.Cu) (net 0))
 (segment (start 100.965 123.695) (end 96.52 119.25) (width 0.25) (layer B.Cu) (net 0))
 (segment (start 100.965 124.445) (end 100.965 123.695) (width 0.25) (layer B.Cu) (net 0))
 (segment (start 96.52 119.25) (end 96.52 100.33) (width 0.25) (layer B.Cu) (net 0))
 (segment (start 96.52 100.33) (end 107.315 100.33) (width 0.25) (layer B.Cu) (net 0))
 (segment (start 107.5 99.375) (end 108 99.375) (width 0.25) (layer B.Cu) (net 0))
 (segment (start 107.315 99.56) (end 107.5 99.375) (width 0.25) (layer B.Cu) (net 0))
 (segment (start 107.315 100.33) (end 107.315 99.56) (width 0.25) (layer B.Cu) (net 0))
 (segment (start 107.5 79.055) (end 107.18 79.375) (width 0.25) (layer B.Cu) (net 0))
 (segment (start 108 79.055) (end 107.5 79.055) (width 0.25) (layer B.Cu) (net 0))
 (segment (start 107.18 79.375) (end 95.25 79.375) (width 0.25) (layer B.Cu) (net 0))
 (segment (start 95.25 79.375) (end 95.25 119.38) (width 0.25) (layer B.Cu) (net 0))
 (segment (start 97.155 121.285) (end 97.155 124.445) (width 0.25) (layer B.Cu) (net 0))
 (segment (start 95.25 119.38) (end 97.155 121.285) (width 0.25) (layer B.Cu) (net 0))
 (segment (start 108 58.735) (end 107 58.735) (width 0.25) (layer B.Cu) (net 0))
 (segment (start 107 58.735) (end 106.68 59.055) (width 0.25) (layer B.Cu) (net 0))
 (segment (start 106.68 59.055) (end 93.98 59.055) (width 0.25) (layer B.Cu) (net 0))
 (segment (start 93.345 59.69) (end 93.345 124.445) (width 0.25) (layer B.Cu) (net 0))
 (segment (start 93.98 59.055) (end 93.345 59.69) (width 0.25) (layer B.Cu) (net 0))
 (segment (start 152.4 123.205) (end 152.4 125.73) (width 0.25) (layer B.Cu) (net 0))
 (segment (start 153.655 120.65) (end 152.4 121.905) (width 0.25) (layer B.Cu) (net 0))
 (segment (start 153.67 120.65) (end 153.655 120.65) (width 0.25) (layer B.Cu) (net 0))
 (segment (start 159.878 114.442) (end 153.67 120.65) (width 0.25) (layer F.Cu) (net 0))
 (segment (start 159.878 110.562) (end 159.878 114.442) (width 0.25) (layer F.Cu) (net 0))
 (segment (start 149.86 123.205) (end 149.86 125.73) (width 0.25) (layer B.Cu) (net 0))
 (via (at 149.86 120.65) (size 0.8) (drill 0.4) (layers F.Cu B.Cu) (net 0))
 (segment (start 147.32 123.955) (end 147.32 125.73) (width 0.25) (layer B.Cu) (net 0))
 (segment (start 147.32 123.205) (end 147.32 123.955) (width 0.25) (layer B.Cu) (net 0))
 (via (at 147.32 120.65) (size 0.8) (drill 0.4) (layers F.Cu B.Cu) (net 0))
 (via (at 143.256 121.92) (size 0.8) (drill 0.4) (layers F.Cu B.Cu) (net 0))
 (segment (start 133.985 112.649) (end 143.256 121.92) (width 0.25) (layer F.Cu) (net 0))
 (segment (start 133.985 112.395) (end 133.985 112.649) (width 0.25) (layer F.Cu) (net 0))
 (segment (start 144.765 121.92) (end 144.78 121.905) (width 0.25) (layer B.Cu) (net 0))
 (segment (start 143.256 121.92) (end 144.765 121.92) (width 0.25) (layer B.Cu) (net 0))
 (segment (start 105.973 110.562) (end 98.918 110.562) (width 0.25) (layer F.Cu) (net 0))
 (segment (start 106.045 110.49) (end 105.973 110.562) (width 0.25) (layer F.Cu) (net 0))
 (segment (start 129.468 110.562) (end 119.238 110.562) (width 0.25) (layer F.Cu) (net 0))
 (segment (start 145.796 119.126) (end 142.748 119.126) (width 0.25) (layer F.Cu) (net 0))
 (segment (start 147.32 120.65) (end 145.796 119.126) (width 0.25) (layer F.Cu) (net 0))
 (segment (start 142.748 117.983) (end 135.327 110.562) (width 0.25) (layer F.Cu) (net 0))
 (segment (start 142.748 119.126) (end 142.748 117.983) (width 0.25) (layer F.Cu) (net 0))
 (segment (start 135.327 110.562) (end 129.468 110.562) (width 0.25) (layer F.Cu) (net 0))
 (segment (start 147.32 120.65) (end 147.32 121.905) (width 0.25) (layer B.Cu) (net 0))
 (segment (start 149.86 120.65) (end 149.86 121.905) (width 0.25) (layer B.Cu) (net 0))
 (segment (start 139.772 110.562) (end 139.558 110.562) (width 0.25) (layer F.Cu) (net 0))
 (segment (start 149.86 120.65) (end 139.772 110.562) (width 0.25) (layer F.Cu) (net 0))
 (segment (start 144.78 123.955) (end 144.78 125.73) (width 0.25) (layer B.Cu) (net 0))
 (segment (start 144.78 123.205) (end 144.78 123.955) (width 0.25) (layer B.Cu) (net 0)))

